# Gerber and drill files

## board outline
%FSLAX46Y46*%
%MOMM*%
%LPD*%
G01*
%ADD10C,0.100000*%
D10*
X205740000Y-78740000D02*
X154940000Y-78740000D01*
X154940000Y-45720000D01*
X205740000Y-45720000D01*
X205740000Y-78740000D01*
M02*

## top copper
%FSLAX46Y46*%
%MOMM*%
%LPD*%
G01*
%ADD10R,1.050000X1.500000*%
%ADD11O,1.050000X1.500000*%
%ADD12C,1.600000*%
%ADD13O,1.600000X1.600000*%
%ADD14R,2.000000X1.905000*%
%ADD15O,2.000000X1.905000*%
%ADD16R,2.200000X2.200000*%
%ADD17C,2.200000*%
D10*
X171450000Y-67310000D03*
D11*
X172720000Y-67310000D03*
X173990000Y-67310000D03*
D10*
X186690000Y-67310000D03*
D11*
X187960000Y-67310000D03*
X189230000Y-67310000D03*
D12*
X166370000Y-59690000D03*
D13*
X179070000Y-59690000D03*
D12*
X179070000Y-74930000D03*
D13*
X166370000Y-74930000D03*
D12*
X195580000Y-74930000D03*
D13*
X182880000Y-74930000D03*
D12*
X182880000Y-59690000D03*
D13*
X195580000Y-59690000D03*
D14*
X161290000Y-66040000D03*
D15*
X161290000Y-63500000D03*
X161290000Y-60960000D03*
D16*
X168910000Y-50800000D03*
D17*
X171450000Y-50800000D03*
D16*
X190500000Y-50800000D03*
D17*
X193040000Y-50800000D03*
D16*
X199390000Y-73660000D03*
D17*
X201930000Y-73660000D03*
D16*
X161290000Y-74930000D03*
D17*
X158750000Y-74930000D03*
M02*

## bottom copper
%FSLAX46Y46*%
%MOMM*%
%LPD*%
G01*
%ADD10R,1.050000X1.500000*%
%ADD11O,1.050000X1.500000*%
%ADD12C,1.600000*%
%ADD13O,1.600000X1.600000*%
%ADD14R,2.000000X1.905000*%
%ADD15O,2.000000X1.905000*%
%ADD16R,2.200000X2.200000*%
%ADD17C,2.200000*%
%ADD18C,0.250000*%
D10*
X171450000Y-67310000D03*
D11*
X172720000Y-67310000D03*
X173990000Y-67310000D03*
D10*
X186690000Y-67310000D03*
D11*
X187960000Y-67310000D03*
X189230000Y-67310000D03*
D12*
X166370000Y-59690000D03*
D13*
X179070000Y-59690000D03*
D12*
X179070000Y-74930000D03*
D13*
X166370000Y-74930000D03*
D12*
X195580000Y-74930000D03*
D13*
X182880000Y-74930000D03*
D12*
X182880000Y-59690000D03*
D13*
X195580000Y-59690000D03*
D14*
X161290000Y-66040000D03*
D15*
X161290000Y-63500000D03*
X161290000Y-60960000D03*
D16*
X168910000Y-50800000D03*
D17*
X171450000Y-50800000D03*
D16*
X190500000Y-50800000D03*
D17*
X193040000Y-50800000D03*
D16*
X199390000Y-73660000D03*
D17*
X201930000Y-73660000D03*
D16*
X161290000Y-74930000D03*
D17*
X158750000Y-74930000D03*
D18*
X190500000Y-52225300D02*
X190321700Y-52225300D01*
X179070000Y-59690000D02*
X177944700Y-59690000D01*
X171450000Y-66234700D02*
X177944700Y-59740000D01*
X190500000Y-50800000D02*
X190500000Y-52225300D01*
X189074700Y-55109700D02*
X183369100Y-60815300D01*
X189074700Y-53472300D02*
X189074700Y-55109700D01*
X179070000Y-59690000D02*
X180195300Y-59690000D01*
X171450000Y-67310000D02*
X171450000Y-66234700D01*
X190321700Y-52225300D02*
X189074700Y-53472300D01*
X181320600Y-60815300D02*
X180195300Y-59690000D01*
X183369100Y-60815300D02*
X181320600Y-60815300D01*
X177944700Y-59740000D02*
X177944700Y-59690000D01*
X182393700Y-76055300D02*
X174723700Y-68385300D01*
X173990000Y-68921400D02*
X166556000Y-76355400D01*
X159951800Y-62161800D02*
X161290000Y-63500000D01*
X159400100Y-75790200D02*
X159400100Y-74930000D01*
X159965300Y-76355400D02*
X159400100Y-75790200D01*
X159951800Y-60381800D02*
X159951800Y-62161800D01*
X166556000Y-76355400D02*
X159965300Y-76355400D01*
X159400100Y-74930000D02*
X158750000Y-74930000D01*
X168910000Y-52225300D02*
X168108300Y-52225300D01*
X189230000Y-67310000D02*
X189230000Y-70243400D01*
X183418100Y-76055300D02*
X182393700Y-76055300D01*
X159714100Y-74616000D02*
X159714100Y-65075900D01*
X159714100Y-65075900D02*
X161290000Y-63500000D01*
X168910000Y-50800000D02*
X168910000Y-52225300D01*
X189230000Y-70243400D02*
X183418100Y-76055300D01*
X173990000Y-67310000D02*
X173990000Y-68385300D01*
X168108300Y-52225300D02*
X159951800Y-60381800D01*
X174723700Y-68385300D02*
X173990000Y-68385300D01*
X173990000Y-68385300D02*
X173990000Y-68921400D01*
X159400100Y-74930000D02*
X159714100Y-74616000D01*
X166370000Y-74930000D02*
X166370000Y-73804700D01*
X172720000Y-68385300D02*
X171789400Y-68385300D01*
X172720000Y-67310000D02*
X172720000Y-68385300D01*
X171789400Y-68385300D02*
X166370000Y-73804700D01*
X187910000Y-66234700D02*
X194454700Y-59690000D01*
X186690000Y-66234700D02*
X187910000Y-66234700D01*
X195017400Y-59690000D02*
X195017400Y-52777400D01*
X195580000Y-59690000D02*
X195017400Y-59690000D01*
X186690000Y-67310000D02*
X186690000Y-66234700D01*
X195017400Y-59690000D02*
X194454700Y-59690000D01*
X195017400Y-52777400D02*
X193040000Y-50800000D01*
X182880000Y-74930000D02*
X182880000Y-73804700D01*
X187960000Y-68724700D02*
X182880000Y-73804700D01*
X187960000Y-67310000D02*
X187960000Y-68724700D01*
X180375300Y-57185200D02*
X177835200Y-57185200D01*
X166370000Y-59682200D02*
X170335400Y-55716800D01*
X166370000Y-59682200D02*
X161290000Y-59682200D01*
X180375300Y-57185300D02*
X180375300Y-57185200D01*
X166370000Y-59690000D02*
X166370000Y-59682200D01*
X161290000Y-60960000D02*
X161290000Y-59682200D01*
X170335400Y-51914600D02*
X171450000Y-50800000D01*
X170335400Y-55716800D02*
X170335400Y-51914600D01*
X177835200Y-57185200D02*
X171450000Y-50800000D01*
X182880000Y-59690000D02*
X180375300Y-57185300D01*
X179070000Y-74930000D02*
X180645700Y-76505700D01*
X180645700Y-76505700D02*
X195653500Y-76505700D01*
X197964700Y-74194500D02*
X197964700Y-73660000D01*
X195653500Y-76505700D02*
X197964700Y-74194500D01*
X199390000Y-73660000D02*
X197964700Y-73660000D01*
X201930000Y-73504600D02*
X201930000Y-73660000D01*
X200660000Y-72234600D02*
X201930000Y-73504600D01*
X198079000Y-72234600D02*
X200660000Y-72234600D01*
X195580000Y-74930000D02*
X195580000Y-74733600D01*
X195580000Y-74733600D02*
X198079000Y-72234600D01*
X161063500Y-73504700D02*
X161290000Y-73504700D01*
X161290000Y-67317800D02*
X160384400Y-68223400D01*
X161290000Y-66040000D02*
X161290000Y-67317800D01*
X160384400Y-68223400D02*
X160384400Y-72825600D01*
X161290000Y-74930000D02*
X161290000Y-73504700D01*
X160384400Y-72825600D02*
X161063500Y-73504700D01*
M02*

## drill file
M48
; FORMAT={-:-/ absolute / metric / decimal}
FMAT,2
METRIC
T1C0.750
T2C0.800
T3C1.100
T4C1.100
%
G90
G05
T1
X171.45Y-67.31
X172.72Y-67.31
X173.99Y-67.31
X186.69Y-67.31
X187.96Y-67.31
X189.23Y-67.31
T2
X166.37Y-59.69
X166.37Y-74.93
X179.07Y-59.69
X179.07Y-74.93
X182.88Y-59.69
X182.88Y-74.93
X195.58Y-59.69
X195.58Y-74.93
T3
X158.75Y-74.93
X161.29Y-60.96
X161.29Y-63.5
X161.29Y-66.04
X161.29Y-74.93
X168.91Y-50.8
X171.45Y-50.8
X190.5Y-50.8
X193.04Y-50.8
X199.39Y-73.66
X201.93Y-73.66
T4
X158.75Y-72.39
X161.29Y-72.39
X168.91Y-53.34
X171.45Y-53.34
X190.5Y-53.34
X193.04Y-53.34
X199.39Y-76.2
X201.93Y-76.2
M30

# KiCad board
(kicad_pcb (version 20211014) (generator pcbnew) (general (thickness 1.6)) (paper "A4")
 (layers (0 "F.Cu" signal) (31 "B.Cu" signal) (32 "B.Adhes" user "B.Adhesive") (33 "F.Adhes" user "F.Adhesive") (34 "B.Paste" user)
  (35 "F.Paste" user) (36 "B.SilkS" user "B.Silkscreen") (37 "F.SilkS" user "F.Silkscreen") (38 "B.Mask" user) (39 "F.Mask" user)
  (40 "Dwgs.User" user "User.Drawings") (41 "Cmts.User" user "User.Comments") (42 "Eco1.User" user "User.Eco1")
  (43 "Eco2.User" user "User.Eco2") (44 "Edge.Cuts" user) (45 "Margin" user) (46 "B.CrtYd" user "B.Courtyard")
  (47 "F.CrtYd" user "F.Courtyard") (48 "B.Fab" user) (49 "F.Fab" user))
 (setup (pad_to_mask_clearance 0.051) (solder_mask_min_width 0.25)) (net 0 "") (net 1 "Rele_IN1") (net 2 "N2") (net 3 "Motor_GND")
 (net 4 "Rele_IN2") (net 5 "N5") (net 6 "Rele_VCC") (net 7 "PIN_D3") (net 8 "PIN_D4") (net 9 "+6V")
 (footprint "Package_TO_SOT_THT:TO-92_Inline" (layer "F.Cu") (at 171.45 67.31)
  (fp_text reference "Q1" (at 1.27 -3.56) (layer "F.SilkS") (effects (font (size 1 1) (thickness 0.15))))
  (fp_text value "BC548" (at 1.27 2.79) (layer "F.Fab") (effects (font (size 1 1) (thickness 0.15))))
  (pad "1" thru_hole rect locked (at 0 0) (size 1.05 1.5) (drill 0.75) (layers *.Cu *.Mask) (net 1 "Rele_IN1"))
  (pad "2" thru_hole oval locked (at 1.27 0) (size 1.05 1.5) (drill 0.75) (layers *.Cu *.Mask) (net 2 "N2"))
  (pad "3" thru_hole oval locked (at 2.54 0) (size 1.05 1.5) (drill 0.75) (layers *.Cu *.Mask) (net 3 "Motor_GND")))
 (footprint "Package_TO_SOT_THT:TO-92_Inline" (layer "F.Cu") (at 186.69 67.31)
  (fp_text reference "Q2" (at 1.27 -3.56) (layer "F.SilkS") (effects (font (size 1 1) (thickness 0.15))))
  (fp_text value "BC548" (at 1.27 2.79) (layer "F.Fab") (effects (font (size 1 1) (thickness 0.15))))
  (pad "1" thru_hole rect locked (at 0 0) (size 1.05 1.5) (drill 0.75) (layers *.Cu *.Mask) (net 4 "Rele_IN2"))
  (pad "2" thru_hole oval locked (at 1.27 0) (size 1.05 1.5) (drill 0.75) (layers *.Cu *.Mask) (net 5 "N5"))
  (pad "3" thru_hole oval locked (at 2.54 0) (size 1.05 1.5) (drill 0.75) (layers *.Cu *.Mask) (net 3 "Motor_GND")))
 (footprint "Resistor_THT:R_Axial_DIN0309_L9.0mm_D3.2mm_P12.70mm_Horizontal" (layer "F.Cu") (at 166.37 59.69)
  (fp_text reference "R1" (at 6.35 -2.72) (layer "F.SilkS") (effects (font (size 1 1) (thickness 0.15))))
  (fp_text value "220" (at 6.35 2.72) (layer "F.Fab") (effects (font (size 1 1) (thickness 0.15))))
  (pad "1" thru_hole circle locked (at 0 0) (size 1.6 1.6) (drill 0.8) (layers *.Cu *.Mask) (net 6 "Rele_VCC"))
  (pad "2" thru_hole oval locked (at 12.7 0) (size 1.6 1.6) (drill 0.8) (layers *.Cu *.Mask) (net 1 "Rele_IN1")))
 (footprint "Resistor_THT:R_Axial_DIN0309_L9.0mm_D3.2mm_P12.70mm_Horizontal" (layer "F.Cu") (at 179.07 74.93 180)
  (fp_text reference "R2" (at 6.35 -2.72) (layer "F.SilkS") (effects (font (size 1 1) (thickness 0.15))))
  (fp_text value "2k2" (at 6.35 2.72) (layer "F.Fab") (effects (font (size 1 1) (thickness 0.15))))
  (pad "1" thru_hole circle locked (at 0 0 180) (size 1.6 1.6) (drill 0.8) (layers *.Cu *.Mask) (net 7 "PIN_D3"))
  (pad "2" thru_hole oval locked (at 12.7 0 180) (size 1.6 1.6) (drill 0.8) (layers *.Cu *.Mask) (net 2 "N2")))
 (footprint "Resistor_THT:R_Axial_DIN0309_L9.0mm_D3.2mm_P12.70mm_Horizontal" (layer "F.Cu") (at 195.58 74.93 180)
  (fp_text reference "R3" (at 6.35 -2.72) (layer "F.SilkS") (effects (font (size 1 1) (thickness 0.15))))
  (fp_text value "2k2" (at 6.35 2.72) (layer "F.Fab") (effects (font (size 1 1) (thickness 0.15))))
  (pad "1" thru_hole circle locked (at 0 0 180) (size 1.6 1.6) (drill 0.8) (layers *.Cu *.Mask) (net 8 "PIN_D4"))
  (pad "2" thru_hole oval locked (at 12.7 0 180) (size 1.6 1.6) (drill 0.8) (layers *.Cu *.Mask) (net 5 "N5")))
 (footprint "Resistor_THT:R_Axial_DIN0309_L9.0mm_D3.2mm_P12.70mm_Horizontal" (layer "F.Cu") (at 182.88 59.69)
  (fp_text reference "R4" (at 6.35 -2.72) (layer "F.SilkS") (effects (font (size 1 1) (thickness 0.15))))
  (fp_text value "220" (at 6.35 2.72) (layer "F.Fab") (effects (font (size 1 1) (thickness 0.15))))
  (pad "1" thru_hole circle locked (at 0 0) (size 1.6 1.6) (drill 0.8) (layers *.Cu *.Mask) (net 6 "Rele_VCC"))
  (pad "2" thru_hole oval locked (at 12.7 0) (size 1.6 1.6) (drill 0.8) (layers *.Cu *.Mask) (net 4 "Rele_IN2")))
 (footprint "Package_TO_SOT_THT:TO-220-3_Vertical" (layer "F.Cu") (at 161.29 66.04 90)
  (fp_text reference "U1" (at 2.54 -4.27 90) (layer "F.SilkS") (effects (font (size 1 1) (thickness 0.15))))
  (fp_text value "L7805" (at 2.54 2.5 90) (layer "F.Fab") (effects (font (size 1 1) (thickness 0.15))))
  (pad "1" thru_hole rect locked (at 0 0 90) (size 1.905 2) (drill 1.1) (layers *.Cu *.Mask) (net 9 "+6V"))
  (pad "2" thru_hole oval locked (at 2.54 0 90) (size 1.905 2) (drill 1.1) (layers *.Cu *.Mask) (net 3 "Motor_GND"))
  (pad "3" thru_hole oval locked (at 5.08 0 90) (size 1.905 2) (drill 1.1) (layers *.Cu *.Mask) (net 6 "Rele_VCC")))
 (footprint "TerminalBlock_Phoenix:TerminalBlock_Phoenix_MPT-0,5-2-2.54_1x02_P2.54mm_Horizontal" (layer "F.Cu") (at 168.91 50.8)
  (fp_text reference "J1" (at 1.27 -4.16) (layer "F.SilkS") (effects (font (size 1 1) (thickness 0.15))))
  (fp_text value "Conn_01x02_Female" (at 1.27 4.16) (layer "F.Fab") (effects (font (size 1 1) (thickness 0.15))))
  (pad "" np_thru_hole circle locked (at 0 2.54) (size 1.1 1.1) (drill 1.1) (layers *.Cu *.Mask))
  (pad "" np_thru_hole circle locked (at 2.54 2.54) (size 1.1 1.1) (drill 1.1) (layers *.Cu *.Mask))
  (pad "1" thru_hole rect locked (at 0 0) (size 2.2 2.2) (drill 1.1) (layers *.Cu *.Mask) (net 3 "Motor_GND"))
  (pad "2" thru_hole circle locked (at 2.54 0) (size 2.2 2.2) (drill 1.1) (layers *.Cu *.Mask) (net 6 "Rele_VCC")))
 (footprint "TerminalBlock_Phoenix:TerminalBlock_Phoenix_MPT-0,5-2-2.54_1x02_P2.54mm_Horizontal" (layer "F.Cu") (at 190.5 50.8)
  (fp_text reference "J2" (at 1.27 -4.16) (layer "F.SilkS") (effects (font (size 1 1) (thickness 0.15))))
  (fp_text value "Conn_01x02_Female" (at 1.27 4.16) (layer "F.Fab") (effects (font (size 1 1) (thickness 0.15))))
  (pad "" np_thru_hole circle locked (at 2.54 2.54) (size 1.1 1.1) (drill 1.1) (layers *.Cu *.Mask))
  (pad "" np_thru_hole circle locked (at 0 2.54) (size 1.1 1.1) (drill 1.1) (layers *.Cu *.Mask))
  (pad "1" thru_hole rect locked (at 0 0) (size 2.2 2.2) (drill 1.1) (layers *.Cu *.Mask) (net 1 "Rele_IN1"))
  (pad "2" thru_hole circle locked (at 2.54 0) (size 2.2 2.2) (drill 1.1) (layers *.Cu *.Mask) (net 4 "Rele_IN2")))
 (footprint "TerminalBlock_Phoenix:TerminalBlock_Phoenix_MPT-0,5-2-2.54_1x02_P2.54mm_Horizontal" (layer "F.Cu") (at 199.39 73.66)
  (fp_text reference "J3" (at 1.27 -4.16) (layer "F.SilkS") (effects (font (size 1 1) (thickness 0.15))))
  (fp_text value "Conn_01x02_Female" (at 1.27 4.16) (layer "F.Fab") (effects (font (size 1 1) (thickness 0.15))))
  (pad "" np_thru_hole circle locked (at 2.54 2.54) (size 1.1 1.1) (drill 1.1) (layers *.Cu *.Mask))
  (pad "" np_thru_hole circle locked (at 0 2.54) (size 1.1 1.1) (drill 1.1) (layers *.Cu *.Mask))
  (pad "1" thru_hole rect locked (at 0 0) (size 2.2 2.2) (drill 1.1) (layers *.Cu *.Mask) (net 7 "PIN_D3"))
  (pad "2" thru_hole circle locked (at 2.54 0) (size 2.2 2.2) (drill 1.1) (layers *.Cu *.Mask) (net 8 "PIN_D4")))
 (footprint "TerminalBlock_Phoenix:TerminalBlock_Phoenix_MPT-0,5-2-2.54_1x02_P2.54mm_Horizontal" (layer "F.Cu") (at 161.29 74.93 180)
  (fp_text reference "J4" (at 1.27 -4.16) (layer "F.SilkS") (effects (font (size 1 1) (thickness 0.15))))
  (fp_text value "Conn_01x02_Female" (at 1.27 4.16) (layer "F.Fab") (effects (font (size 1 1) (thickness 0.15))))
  (pad "" np_thru_hole circle locked (at 2.54 2.54 180) (size 1.1 1.1) (drill 1.1) (layers *.Cu *.Mask))
  (pad "" np_thru_hole circle locked (at 0 2.54 180) (size 1.1 1.1) (drill 1.1) (layers *.Cu *.Mask))
  (pad "1" thru_hole rect locked (at 0 0 180) (size 2.2 2.2) (drill 1.1) (layers *.Cu *.Mask) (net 9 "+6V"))
  (pad "2" thru_hole circle locked (at 2.54 0 180) (size 2.2 2.2) (drill 1.1) (layers *.Cu *.Mask) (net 3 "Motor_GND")))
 (gr_poly (pts (xy 205.74 78.74) (xy 154.94 78.74) (xy 154.94 45.72) (xy 205.74 45.72)) (layer "Edge.Cuts") (width 0.1) (fill none))
 (segment (start 190.5 52.2253) (end 190.3217 52.2253) (width 0.25) (layer "B.Cu") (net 1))
 (segment (start 179.07 59.69) (end 177.9447 59.69) (width 0.25) (layer "B.Cu") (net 1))
 (segment (start 171.45 66.2347) (end 177.9447 59.74) (width 0.25) (layer "B.Cu") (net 1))
 (segment (start 190.5 50.8) (end 190.5 52.2253) (width 0.25) (layer "B.Cu") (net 1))
 (segment (start 189.0747 55.1097) (end 183.3691 60.8153) (width 0.25) (layer "B.Cu") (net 1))
 (segment (start 189.0747 53.4723) (end 189.0747 55.1097) (width 0.25) (layer "B.Cu") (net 1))
 (segment (start 179.07 59.69) (end 180.1953 59.69) (width 0.25) (layer "B.Cu") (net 1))
 (segment (start 171.45 67.31) (end 171.45 66.2347) (width 0.25) (layer "B.Cu") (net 1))
 (segment (start 190.3217 52.2253) (end 189.0747 53.4723) (width 0.25) (layer "B.Cu") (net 1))
 (segment (start 181.3206 60.8153) (end 180.1953 59.69) (width 0.25) (layer "B.Cu") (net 1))
 (segment (start 183.3691 60.8153) (end 181.3206 60.8153) (width 0.25) (layer "B.Cu") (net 1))
 (segment (start 177.9447 59.74) (end 177.9447 59.69) (width 0.25) (layer "B.Cu") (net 1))
 (segment (start 182.3937 76.0553) (end 174.7237 68.3853) (width 0.25) (layer "B.Cu") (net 3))
 (segment (start 173.99 68.9214) (end 166.556 76.3554) (width 0.25) (layer "B.Cu") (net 3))
 (segment (start 159.9518 62.1618) (end 161.29 63.5) (width 0.25) (layer "B.Cu") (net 3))
 (segment (start 159.4001 75.7902) (end 159.4001 74.93) (width 0.25) (layer "B.Cu") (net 3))
 (segment (start 159.9653 76.3554) (end 159.4001 75.7902) (width 0.25) (layer "B.Cu") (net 3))
 (segment (start 159.9518 60.3818) (end 159.9518 62.1618) (width 0.25) (layer "B.Cu") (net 3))
 (segment (start 166.556 76.3554) (end 159.9653 76.3554) (width 0.25) (layer "B.Cu") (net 3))
 (segment (start 159.4001 74.93) (end 158.75 74.93) (width 0.25) (layer "B.Cu") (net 3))
 (segment (start 168.91 52.2253) (end 168.1083 52.2253) (width 0.25) (layer "B.Cu") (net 3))
 (segment (start 189.23 67.31) (end 189.23 70.2434) (width 0.25) (layer "B.Cu") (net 3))
 (segment (start 183.4181 76.0553) (end 182.3937 76.0553) (width 0.25) (layer "B.Cu") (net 3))
 (segment (start 159.7141 74.616) (end 159.7141 65.0759) (width 0.25) (layer "B.Cu") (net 3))
 (segment (start 159.7141 65.0759) (end 161.29 63.5) (width 0.25) (layer "B.Cu") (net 3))
 (segment (start 168.91 50.8) (end 168.91 52.2253) (width 0.25) (layer "B.Cu") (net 3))
 (segment (start 189.23 70.2434) (end 183.4181 76.0553) (width 0.25) (layer "B.Cu") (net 3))
 (segment (start 173.99 67.31) (end 173.99 68.3853) (width 0.25) (layer "B.Cu") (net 3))
 (segment (start 168.1083 52.2253) (end 159.9518 60.3818) (width 0.25) (layer "B.Cu") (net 3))
 (segment (start 174.7237 68.3853) (end 173.99 68.3853) (width 0.25) (layer "B.Cu") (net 3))
 (segment (start 173.99 68.3853) (end 173.99 68.9214) (width 0.25) (layer "B.Cu") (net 3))
 (segment (start 159.4001 74.93) (end 159.7141 74.616) (width 0.25) (layer "B.Cu") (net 3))
 (segment (start 166.37 74.93) (end 166.37 73.8047) (width 0.25) (layer "B.Cu") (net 2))
 (segment (start 172.72 68.3853) (end 171.7894 68.3853) (width 0.25) (layer "B.Cu") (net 2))
 (segment (start 172.72 67.31) (end 172.72 68.3853) (width 0.25) (layer "B.Cu") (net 2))
 (segment (start 171.7894 68.3853) (end 166.37 73.8047) (width 0.25) (layer "B.Cu") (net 2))
 (segment (start 187.91 66.2347) (end 194.4547 59.69) (width 0.25) (layer "B.Cu") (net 4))
 (segment (start 186.69 66.2347) (end 187.91 66.2347) (width 0.25) (layer "B.Cu") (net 4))
 (segment (start 195.0174 59.69) (end 195.0174 52.7774) (width 0.25) (layer "B.Cu") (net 4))
 (segment (start 195.58 59.69) (end 195.0174 59.69) (width 0.25) (layer "B.Cu") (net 4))
 (segment (start 186.69 67.31) (end 186.69 66.2347) (width 0.25) (layer "B.Cu") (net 4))
 (segment (start 195.0174 59.69) (end 194.4547 59.69) (width 0.25) (layer "B.Cu") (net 4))
 (segment (start 195.0174 52.7774) (end 193.04 50.8) (width 0.25) (layer "B.Cu") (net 4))
 (segment (start 182.88 74.93) (end 182.88 73.8047) (width 0.25) (layer "B.Cu") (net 5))
 (segment (start 187.96 68.7247) (end 182.88 73.8047) (width 0.25) (layer "B.Cu") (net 5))
 (segment (start 187.96 67.31) (end 187.96 68.7247) (width 0.25) (layer "B.Cu") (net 5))
 (segment (start 180.3753 57.1852) (end 177.8352 57.1852) (width 0.25) (layer "B.Cu") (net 6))
 (segment (start 166.37 59.6822) (end 170.3354 55.7168) (width 0.25) (layer "B.Cu") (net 6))
 (segment (start 166.37 59.6822) (end 161.29 59.6822) (width 0.25) (layer "B.Cu") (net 6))
 (segment (start 180.3753 57.1853) (end 180.3753 57.1852) (width 0.25) (layer "B.Cu") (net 6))
 (segment (start 166.37 59.69) (end 166.37 59.6822) (width 0.25) (layer "B.Cu") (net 6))
 (segment (start 161.29 60.96) (end 161.29 59.6822) (width 0.25) (layer "B.Cu") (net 6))
 (segment (start 170.3354 51.9146) (end 171.45 50.8) (width 0.25) (layer "B.Cu") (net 6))
 (segment (start 170.3354 55.7168) (end 170.3354 51.9146) (width 0.25) (layer "B.Cu") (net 6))
 (segment (start 177.8352 57.1852) (end 171.45 50.8) (width 0.25) (layer "B.Cu") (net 6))
 (segment (start 182.88 59.69) (end 180.3753 57.1853) (width 0.25) (layer "B.Cu") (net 6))
 (segment (start 179.07 74.93) (end 180.6457 76.5057) (width 0.25) (layer "B.Cu") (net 7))
 (segment (start 180.6457 76.5057) (end 195.6535 76.5057) (width 0.25) (layer "B.Cu") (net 7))
 (segment (start 197.9647 74.1945) (end 197.9647 73.66) (width 0.25) (layer "B.Cu") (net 7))
 (segment (start 195.6535 76.5057) (end 197.9647 74.1945) (width 0.25) (layer "B.Cu") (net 7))
 (segment (start 199.39 73.66) (end 197.9647 73.66) (width 0.25) (layer "B.Cu") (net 7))
 (segment (start 201.93 73.5046) (end 201.93 73.66) (width 0.25) (layer "B.Cu") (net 8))
 (segment (start 200.66 72.2346) (end 201.93 73.5046) (width 0.25) (layer "B.Cu") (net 8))
 (segment (start 198.079 72.2346) (end 200.66 72.2346) (width 0.25) (layer "B.Cu") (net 8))
 (segment (start 195.58 74.93) (end 195.58 74.7336) (width 0.25) (layer "B.Cu") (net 8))
 (segment (start 195.58 74.7336) (end 198.079 72.2346) (width 0.25) (layer "B.Cu") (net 8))
 (segment (start 161.0635 73.5047) (end 161.29 73.5047) (width 0.25) (layer "B.Cu") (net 9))
 (segment (start 161.29 67.3178) (end 160.3844 68.2234) (width 0.25) (layer "B.Cu") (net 9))
 (segment (start 161.29 66.04) (end 161.29 67.3178) (width 0.25) (layer "B.Cu") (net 9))
 (segment (start 160.3844 68.2234) (end 160.3844 72.8256) (width 0.25) (layer "B.Cu") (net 9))
 (segment (start 161.29 74.93) (end 161.29 73.5047) (width 0.25) (layer "B.Cu") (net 9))
 (segment (start 160.3844 72.8256) (end 161.0635 73.5047) (width 0.25) (layer "B.Cu") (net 9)))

